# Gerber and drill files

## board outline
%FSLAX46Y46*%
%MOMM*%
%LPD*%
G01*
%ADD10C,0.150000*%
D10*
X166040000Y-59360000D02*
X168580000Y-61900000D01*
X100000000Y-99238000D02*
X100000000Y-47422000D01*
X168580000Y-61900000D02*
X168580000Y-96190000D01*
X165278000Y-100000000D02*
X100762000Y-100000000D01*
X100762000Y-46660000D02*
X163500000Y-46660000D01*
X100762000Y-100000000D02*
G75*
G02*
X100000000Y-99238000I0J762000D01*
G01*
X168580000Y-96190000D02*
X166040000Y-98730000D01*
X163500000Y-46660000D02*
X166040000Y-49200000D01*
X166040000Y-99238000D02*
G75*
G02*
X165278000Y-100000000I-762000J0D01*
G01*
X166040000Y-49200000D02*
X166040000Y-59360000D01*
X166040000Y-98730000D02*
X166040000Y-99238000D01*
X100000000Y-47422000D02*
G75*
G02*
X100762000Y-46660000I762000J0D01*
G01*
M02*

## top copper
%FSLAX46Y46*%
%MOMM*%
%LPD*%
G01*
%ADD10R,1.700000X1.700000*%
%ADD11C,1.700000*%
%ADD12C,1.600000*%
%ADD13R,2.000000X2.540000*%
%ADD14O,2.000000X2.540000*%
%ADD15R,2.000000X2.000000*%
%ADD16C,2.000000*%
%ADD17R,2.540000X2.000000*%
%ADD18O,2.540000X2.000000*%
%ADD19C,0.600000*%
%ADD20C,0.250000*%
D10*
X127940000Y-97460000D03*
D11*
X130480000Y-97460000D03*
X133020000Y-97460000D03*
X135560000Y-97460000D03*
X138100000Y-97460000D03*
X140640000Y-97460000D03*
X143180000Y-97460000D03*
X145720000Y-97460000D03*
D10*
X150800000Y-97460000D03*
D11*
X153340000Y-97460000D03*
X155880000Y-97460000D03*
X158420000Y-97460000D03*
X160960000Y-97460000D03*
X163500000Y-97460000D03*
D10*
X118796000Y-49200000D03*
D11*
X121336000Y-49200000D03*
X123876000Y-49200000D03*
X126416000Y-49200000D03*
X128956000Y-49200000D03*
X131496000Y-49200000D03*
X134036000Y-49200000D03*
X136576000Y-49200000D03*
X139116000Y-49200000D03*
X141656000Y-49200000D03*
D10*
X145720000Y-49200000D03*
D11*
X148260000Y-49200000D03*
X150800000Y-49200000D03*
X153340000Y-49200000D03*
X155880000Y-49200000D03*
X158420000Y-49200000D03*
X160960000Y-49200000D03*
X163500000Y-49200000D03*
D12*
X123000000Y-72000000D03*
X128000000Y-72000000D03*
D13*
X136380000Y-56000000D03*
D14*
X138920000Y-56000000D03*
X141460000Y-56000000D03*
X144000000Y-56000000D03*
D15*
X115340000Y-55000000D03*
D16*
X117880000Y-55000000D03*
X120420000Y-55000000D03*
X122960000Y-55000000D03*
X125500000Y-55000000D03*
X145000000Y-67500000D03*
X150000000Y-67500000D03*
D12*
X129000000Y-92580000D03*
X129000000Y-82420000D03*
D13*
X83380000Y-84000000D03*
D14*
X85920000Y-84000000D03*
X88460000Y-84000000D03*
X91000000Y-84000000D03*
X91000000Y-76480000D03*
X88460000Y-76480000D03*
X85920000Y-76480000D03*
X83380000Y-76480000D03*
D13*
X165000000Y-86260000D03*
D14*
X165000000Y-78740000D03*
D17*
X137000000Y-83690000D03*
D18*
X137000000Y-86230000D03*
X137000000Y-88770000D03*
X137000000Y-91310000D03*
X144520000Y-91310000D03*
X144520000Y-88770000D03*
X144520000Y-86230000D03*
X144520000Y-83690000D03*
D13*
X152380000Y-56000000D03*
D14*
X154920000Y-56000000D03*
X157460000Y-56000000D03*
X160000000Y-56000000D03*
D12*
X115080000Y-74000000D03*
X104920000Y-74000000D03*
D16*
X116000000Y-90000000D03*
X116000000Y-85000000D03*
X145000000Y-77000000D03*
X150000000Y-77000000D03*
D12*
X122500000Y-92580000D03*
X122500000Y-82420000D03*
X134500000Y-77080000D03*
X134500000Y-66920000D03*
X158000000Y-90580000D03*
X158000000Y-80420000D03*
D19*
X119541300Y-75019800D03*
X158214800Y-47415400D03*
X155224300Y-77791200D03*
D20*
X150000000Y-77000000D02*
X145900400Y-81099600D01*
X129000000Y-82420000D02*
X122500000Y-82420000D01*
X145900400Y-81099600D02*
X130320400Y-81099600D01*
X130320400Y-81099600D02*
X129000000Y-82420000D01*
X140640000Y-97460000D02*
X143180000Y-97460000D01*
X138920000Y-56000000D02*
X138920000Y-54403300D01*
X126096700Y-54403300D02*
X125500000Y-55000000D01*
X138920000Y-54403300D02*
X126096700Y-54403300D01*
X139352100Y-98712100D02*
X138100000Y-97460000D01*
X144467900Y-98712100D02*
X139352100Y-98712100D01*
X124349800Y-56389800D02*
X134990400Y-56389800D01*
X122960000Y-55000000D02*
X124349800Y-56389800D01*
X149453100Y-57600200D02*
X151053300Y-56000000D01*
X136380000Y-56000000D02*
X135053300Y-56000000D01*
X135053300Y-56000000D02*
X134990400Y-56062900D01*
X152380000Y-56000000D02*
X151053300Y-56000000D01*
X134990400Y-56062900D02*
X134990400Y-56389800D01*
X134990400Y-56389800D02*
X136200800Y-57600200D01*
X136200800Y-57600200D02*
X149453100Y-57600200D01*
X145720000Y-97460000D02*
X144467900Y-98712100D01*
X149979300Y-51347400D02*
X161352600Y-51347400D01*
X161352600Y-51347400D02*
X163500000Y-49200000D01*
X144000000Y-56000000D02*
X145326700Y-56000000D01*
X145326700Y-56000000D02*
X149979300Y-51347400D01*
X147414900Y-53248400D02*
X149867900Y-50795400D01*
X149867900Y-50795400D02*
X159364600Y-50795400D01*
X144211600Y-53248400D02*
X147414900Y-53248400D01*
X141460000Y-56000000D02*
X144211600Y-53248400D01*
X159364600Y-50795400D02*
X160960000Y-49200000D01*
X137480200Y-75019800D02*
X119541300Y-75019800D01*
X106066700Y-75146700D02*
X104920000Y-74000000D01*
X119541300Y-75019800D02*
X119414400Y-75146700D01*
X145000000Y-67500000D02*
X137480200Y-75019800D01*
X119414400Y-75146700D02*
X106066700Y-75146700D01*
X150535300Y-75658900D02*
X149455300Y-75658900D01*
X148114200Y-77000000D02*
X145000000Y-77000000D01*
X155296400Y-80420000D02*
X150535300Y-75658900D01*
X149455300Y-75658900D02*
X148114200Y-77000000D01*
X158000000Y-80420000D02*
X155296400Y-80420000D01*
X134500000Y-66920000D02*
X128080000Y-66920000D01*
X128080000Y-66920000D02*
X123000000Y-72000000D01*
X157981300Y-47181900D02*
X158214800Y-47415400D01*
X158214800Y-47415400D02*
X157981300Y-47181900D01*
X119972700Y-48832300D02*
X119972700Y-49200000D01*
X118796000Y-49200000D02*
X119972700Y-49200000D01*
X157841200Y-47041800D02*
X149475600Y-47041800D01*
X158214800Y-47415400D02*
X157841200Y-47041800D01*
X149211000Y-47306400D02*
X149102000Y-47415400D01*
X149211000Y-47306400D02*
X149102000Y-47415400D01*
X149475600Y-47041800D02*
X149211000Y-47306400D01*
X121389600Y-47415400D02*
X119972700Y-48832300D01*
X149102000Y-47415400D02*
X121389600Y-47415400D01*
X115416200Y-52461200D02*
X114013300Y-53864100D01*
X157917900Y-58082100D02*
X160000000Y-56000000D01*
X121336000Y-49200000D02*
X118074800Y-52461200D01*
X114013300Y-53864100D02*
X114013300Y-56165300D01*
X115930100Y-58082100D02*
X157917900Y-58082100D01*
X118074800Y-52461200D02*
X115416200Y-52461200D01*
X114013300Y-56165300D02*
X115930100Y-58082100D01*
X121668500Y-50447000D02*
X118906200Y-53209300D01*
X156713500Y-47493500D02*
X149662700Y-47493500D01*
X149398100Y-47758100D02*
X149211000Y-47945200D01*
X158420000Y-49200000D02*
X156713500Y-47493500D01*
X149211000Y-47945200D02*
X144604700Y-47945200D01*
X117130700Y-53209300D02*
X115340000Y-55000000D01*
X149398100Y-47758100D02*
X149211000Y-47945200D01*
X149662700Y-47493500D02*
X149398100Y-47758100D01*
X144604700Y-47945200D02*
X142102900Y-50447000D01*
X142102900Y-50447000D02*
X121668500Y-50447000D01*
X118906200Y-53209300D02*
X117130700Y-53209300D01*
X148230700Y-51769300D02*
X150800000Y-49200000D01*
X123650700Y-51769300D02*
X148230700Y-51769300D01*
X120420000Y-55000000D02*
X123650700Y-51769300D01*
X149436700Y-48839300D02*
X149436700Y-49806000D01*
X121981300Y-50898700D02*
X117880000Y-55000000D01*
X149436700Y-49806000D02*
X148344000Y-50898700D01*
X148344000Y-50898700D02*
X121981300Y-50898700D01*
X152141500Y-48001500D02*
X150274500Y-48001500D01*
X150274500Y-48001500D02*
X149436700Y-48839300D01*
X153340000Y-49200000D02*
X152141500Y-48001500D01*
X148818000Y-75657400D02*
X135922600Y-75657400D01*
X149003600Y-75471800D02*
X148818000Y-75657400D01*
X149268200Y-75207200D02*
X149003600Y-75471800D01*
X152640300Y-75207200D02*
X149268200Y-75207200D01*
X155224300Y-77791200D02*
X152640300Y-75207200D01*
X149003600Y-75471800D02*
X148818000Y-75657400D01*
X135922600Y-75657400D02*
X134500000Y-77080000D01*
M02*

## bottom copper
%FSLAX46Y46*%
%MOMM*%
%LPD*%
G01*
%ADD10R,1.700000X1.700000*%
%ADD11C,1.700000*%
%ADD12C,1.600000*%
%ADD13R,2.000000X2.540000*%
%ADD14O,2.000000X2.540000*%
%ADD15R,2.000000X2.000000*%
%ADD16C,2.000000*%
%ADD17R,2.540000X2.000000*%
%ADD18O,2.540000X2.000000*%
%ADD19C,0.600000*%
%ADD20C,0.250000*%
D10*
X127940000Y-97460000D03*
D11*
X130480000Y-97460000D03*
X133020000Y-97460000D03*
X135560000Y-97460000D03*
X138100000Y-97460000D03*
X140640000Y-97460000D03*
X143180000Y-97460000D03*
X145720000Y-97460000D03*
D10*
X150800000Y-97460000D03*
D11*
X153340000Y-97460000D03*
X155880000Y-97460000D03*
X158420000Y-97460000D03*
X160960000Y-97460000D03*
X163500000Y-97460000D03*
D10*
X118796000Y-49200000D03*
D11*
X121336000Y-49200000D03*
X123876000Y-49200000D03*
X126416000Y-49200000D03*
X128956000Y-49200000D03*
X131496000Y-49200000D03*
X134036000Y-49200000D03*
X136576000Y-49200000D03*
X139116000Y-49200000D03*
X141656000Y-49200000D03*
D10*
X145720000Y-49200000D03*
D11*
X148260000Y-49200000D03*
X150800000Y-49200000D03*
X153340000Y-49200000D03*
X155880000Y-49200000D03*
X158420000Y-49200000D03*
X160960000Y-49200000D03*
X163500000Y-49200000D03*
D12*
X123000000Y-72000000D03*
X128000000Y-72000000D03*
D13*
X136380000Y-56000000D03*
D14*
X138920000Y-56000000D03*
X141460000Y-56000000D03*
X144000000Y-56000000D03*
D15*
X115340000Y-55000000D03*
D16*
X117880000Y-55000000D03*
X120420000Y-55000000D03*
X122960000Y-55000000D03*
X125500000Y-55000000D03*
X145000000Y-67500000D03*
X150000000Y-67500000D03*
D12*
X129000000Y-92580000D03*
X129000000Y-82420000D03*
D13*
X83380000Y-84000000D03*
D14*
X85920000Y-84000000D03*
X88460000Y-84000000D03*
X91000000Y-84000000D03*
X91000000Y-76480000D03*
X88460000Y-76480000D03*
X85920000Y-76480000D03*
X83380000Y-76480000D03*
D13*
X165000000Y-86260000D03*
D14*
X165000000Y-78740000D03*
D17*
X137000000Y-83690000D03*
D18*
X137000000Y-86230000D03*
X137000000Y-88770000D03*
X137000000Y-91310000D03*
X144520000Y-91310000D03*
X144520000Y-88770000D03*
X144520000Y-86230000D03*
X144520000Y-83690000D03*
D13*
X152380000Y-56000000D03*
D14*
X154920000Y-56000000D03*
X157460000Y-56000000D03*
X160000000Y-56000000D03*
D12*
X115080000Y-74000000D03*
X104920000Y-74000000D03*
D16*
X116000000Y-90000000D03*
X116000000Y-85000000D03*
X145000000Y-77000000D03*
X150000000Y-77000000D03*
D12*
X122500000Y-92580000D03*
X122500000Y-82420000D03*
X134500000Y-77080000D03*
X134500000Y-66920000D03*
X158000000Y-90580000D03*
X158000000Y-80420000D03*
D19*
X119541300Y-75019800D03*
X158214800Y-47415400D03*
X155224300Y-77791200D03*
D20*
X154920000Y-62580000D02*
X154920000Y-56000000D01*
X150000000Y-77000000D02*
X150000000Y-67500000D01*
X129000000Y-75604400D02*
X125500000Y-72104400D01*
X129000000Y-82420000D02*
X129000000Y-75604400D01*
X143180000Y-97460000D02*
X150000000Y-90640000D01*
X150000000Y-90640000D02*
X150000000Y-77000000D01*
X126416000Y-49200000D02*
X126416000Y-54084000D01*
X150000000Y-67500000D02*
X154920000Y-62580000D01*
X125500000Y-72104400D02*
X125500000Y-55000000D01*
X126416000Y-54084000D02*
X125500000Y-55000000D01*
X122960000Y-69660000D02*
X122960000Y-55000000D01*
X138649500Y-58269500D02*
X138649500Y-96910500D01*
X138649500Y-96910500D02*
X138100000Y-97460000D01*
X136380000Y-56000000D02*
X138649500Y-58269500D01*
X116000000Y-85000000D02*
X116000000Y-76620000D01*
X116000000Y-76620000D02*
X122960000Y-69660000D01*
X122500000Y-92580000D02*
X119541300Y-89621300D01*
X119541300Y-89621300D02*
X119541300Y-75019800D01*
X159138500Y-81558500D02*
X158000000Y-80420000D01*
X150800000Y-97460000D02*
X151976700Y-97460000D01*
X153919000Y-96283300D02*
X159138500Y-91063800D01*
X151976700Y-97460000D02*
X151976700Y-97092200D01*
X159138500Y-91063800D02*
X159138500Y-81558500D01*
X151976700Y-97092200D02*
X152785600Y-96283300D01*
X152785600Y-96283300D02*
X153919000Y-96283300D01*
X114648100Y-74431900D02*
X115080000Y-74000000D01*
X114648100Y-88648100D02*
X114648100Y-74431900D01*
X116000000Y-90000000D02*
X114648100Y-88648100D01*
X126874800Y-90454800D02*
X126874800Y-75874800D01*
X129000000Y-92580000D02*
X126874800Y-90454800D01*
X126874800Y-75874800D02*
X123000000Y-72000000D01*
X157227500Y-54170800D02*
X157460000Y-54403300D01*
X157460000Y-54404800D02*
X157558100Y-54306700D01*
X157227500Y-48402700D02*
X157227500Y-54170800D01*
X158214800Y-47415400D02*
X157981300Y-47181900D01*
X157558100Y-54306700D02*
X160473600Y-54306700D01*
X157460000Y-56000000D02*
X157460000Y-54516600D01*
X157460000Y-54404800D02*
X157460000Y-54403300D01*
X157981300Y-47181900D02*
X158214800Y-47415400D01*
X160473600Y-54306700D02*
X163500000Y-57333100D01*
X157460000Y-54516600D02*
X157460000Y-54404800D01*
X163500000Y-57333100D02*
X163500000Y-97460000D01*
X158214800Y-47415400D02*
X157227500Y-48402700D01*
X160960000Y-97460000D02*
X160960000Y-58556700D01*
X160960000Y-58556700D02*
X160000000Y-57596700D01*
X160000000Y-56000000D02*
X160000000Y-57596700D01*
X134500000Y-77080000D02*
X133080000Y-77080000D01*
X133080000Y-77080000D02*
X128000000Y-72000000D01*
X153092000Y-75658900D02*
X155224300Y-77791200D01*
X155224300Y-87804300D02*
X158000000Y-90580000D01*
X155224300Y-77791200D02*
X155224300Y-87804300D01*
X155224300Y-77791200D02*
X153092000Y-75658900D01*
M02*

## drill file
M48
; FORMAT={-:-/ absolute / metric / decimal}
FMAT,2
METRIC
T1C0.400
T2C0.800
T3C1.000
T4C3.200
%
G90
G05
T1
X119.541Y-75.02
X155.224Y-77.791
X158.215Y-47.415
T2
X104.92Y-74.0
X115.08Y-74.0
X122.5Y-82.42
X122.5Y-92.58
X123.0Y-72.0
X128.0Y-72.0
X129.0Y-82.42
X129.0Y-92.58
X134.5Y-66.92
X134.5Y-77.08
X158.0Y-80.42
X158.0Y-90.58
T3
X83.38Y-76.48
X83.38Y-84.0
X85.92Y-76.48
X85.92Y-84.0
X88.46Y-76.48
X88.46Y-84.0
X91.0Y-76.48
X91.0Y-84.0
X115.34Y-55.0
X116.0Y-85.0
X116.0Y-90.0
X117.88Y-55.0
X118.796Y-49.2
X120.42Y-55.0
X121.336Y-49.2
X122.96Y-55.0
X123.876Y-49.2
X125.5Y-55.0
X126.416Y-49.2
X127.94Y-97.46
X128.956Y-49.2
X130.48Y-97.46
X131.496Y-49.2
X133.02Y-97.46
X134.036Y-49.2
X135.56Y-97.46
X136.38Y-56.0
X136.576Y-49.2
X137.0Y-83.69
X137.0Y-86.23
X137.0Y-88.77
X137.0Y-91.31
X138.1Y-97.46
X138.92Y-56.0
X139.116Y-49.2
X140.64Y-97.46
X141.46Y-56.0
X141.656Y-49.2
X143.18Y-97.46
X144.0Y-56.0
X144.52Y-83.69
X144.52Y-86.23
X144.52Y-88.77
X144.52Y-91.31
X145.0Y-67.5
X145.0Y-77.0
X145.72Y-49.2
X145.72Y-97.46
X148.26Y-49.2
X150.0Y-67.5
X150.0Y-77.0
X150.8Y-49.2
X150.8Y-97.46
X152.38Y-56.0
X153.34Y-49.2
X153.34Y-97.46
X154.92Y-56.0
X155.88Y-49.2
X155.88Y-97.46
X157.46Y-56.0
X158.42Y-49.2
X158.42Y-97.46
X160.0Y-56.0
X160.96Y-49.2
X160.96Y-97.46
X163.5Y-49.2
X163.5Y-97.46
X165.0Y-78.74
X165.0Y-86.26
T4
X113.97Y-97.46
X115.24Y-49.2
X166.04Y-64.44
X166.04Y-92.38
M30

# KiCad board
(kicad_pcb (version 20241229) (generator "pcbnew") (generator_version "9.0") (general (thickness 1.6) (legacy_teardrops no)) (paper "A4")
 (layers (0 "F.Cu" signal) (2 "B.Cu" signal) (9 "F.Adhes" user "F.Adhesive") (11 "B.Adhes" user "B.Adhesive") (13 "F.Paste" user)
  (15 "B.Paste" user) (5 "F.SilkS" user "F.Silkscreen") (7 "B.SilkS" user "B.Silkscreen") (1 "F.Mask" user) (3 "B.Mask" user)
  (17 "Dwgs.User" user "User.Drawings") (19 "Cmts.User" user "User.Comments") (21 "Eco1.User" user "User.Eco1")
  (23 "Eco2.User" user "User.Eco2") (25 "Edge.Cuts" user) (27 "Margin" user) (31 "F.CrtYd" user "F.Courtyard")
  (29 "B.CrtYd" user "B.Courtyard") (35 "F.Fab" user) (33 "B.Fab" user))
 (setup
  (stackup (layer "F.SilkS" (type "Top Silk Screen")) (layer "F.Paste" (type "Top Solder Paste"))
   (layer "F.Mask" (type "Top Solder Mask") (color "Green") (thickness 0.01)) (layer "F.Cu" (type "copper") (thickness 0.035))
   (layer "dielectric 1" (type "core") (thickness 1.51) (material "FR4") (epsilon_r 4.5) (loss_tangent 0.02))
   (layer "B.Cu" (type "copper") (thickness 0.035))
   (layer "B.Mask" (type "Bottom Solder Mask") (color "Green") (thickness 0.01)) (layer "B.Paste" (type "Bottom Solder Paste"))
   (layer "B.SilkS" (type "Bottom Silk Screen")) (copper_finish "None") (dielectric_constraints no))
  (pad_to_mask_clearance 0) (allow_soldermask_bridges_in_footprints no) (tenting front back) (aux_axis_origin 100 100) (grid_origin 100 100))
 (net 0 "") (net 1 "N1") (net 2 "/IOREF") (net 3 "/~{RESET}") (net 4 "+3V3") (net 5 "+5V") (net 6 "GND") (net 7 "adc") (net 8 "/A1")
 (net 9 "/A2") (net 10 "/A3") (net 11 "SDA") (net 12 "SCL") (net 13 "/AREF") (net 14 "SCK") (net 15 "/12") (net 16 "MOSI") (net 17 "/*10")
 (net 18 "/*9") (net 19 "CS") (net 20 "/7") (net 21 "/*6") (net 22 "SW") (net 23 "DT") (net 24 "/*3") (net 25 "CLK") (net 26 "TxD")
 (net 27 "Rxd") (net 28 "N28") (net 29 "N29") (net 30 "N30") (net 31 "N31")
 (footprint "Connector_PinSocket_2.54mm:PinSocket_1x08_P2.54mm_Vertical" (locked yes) (layer "F.Cu") (at 127.94 97.46 90)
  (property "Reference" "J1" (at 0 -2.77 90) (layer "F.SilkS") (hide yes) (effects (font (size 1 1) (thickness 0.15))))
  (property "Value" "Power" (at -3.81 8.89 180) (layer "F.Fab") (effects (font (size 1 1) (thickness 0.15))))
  (pad "1" thru_hole rect (at 0 0 90) (size 1.7 1.7) (drill 1) (layers "*.Cu" "*.Mask") (remove_unused_layers no) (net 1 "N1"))
  (pad "2" thru_hole circle (at 0 2.54 90) (size 1.7 1.7) (drill 1) (layers "*.Cu" "*.Mask") (remove_unused_layers no) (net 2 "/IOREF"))
  (pad "3" thru_hole circle (at 0 5.08 90) (size 1.7 1.7) (drill 1) (layers "*.Cu" "*.Mask") (remove_unused_layers no) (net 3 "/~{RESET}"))
  (pad "4" thru_hole circle (at 0 7.62 90) (size 1.7 1.7) (drill 1) (layers "*.Cu" "*.Mask") (remove_unused_layers no) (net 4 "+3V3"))
  (pad "5" thru_hole circle (at 0 10.16 90) (size 1.7 1.7) (drill 1) (layers "*.Cu" "*.Mask") (remove_unused_layers no) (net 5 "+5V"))
  (pad "6" thru_hole circle (at 0 12.7 90) (size 1.7 1.7) (drill 1) (layers "*.Cu" "*.Mask") (remove_unused_layers no) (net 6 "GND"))
  (pad "7" thru_hole circle (at 0 15.24 90) (size 1.7 1.7) (drill 1) (layers "*.Cu" "*.Mask") (remove_unused_layers no) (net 6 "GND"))
  (pad "8" thru_hole circle (at 0 17.78 90) (size 1.7 1.7) (drill 1) (layers "*.Cu" "*.Mask") (remove_unused_layers no) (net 5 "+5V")))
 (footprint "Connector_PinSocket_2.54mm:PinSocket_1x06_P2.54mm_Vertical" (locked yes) (layer "F.Cu") (at 150.8 97.46 90)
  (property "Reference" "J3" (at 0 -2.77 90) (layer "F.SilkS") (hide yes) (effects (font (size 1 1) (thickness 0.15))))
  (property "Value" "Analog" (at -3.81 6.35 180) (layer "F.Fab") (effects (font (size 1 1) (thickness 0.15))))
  (pad "1" thru_hole rect (at 0 0 90) (size 1.7 1.7) (drill 1) (layers "*.Cu" "*.Mask") (remove_unused_layers no) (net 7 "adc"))
  (pad "2" thru_hole circle (at 0 2.54 90) (size 1.7 1.7) (drill 1) (layers "*.Cu" "*.Mask") (remove_unused_layers no) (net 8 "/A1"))
  (pad "3" thru_hole circle (at 0 5.08 90) (size 1.7 1.7) (drill 1) (layers "*.Cu" "*.Mask") (remove_unused_layers no) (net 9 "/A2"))
  (pad "4" thru_hole circle (at 0 7.62 90) (size 1.7 1.7) (drill 1) (layers "*.Cu" "*.Mask") (remove_unused_layers no) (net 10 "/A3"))
  (pad "5" thru_hole circle (at 0 10.16 90) (size 1.7 1.7) (drill 1) (layers "*.Cu" "*.Mask") (remove_unused_layers no) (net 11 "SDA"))
  (pad "6" thru_hole circle (at 0 12.7 90) (size 1.7 1.7) (drill 1) (layers "*.Cu" "*.Mask") (remove_unused_layers no) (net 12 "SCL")))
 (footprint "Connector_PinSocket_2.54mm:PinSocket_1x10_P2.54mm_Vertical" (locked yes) (layer "F.Cu") (at 118.796 49.2 90)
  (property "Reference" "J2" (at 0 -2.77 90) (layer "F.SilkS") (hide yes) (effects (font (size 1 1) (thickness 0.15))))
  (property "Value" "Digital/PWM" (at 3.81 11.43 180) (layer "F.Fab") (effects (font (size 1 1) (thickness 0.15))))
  (pad "1" thru_hole rect (at 0 0 90) (size 1.7 1.7) (drill 1) (layers "*.Cu" "*.Mask") (remove_unused_layers no) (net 12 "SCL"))
  (pad "2" thru_hole circle (at 0 2.54 90) (size 1.7 1.7) (drill 1) (layers "*.Cu" "*.Mask") (remove_unused_layers no) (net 11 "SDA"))
  (pad "3" thru_hole circle (at 0 5.08 90) (size 1.7 1.7) (drill 1) (layers "*.Cu" "*.Mask") (remove_unused_layers no) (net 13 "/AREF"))
  (pad "4" thru_hole circle (at 0 7.62 90) (size 1.7 1.7) (drill 1) (layers "*.Cu" "*.Mask") (remove_unused_layers no) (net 6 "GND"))
  (pad "5" thru_hole circle (at 0 10.16 90) (size 1.7 1.7) (drill 1) (layers "*.Cu" "*.Mask") (remove_unused_layers no) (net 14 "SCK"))
  (pad "6" thru_hole circle (at 0 12.7 90) (size 1.7 1.7) (drill 1) (layers "*.Cu" "*.Mask") (remove_unused_layers no) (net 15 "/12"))
  (pad "7" thru_hole circle (at 0 15.24 90) (size 1.7 1.7) (drill 1) (layers "*.Cu" "*.Mask") (remove_unused_layers no) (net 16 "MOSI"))
  (pad "8" thru_hole circle (at 0 17.78 90) (size 1.7 1.7) (drill 1) (layers "*.Cu" "*.Mask") (remove_unused_layers no) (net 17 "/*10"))
  (pad "9" thru_hole circle (at 0 20.32 90) (size 1.7 1.7) (drill 1) (layers "*.Cu" "*.Mask") (remove_unused_layers no) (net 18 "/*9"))
  (pad "10" thru_hole circle (at 0 22.86 90) (size 1.7 1.7) (drill 1) (layers "*.Cu" "*.Mask") (remove_unused_layers no) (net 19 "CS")))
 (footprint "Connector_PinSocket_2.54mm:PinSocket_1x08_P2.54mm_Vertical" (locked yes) (layer "F.Cu") (at 145.72 49.2 90)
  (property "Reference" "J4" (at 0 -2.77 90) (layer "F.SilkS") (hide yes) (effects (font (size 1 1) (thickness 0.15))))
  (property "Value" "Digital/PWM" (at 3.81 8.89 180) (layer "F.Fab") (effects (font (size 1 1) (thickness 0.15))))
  (pad "1" thru_hole rect (at 0 0 90) (size 1.7 1.7) (drill 1) (layers "*.Cu" "*.Mask") (remove_unused_layers no) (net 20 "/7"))
  (pad "2" thru_hole circle (at 0 2.54 90) (size 1.7 1.7) (drill 1) (layers "*.Cu" "*.Mask") (remove_unused_layers no) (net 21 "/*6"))
  (pad "3" thru_hole circle (at 0 5.08 90) (size 1.7 1.7) (drill 1) (layers "*.Cu" "*.Mask") (remove_unused_layers no) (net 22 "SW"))
  (pad "4" thru_hole circle (at 0 7.62 90) (size 1.7 1.7) (drill 1) (layers "*.Cu" "*.Mask") (remove_unused_layers no) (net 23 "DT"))
  (pad "5" thru_hole circle (at 0 10.16 90) (size 1.7 1.7) (drill 1) (layers "*.Cu" "*.Mask") (remove_unused_layers no) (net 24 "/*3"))
  (pad "6" thru_hole circle (at 0 12.7 90) (size 1.7 1.7) (drill 1) (layers "*.Cu" "*.Mask") (remove_unused_layers no) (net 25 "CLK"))
  (pad "7" thru_hole circle (at 0 15.24 90) (size 1.7 1.7) (drill 1) (layers "*.Cu" "*.Mask") (remove_unused_layers no) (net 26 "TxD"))
  (pad "8" thru_hole circle (at 0 17.78 90) (size 1.7 1.7) (drill 1) (layers "*.Cu" "*.Mask") (remove_unused_layers no) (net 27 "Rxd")))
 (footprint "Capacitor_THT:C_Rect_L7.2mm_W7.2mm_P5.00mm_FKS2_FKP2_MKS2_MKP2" (layer "F.Cu") (at 123 72)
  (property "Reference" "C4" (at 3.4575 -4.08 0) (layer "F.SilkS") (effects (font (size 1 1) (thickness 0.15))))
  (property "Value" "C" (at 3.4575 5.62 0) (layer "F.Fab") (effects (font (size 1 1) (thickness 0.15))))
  (pad "1" thru_hole circle (at 0 0) (size 1.6 1.6) (drill 0.8) (layers "*.Cu" "*.Mask") (remove_unused_layers no) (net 6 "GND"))
  (pad "2" thru_hole circle (at 5 0) (size 1.6 1.6) (drill 0.8) (layers "*.Cu" "*.Mask") (remove_unused_layers no) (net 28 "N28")))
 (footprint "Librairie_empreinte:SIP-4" (layer "F.Cu") (at 140.19 56)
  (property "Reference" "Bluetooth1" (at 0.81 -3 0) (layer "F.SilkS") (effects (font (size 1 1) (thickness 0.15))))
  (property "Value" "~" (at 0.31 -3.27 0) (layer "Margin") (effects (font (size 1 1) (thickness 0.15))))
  (pad "1" thru_hole rect (at -3.81 0) (size 2 2.54) (drill 1) (layers "*.Cu" "*.Mask") (remove_unused_layers no) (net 5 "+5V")
   (thermal_bridge_angle 45))
  (pad "2" thru_hole oval (at -1.27 0) (size 2 2.54) (drill 1) (layers "*.Cu" "*.Mask") (remove_unused_layers no) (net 6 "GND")
   (thermal_bridge_angle 45))
  (pad "3" thru_hole oval (at 1.27 0) (size 2 2.54) (drill 1) (layers "*.Cu" "*.Mask") (remove_unused_layers no) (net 26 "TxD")
   (thermal_bridge_angle 45))
  (pad "4" thru_hole oval (at 3.81 0) (size 2 2.54) (drill 1) (layers "*.Cu" "*.Mask") (remove_unused_layers no) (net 27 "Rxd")
   (thermal_bridge_angle 45)))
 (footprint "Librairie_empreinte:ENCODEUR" (layer "F.Cu") (at 120.42 55)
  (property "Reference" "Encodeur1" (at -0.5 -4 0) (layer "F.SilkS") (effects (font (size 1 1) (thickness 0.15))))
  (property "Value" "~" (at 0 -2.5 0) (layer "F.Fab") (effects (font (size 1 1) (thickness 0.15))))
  (pad "1" thru_hole rect (at -5.08 0) (size 2 2) (drill 1) (layers "*.Cu" "*.Mask") (remove_unused_layers no) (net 25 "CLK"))
  (pad "2" thru_hole circle (at -2.54 0) (size 2 2) (drill 1) (layers "*.Cu" "*.Mask") (remove_unused_layers no) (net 23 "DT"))
  (pad "3" thru_hole circle (at 0 0) (size 2 2) (drill 1) (layers "*.Cu" "*.Mask") (remove_unused_layers no) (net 22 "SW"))
  (pad "4" thru_hole circle (at 2.54 0) (size 2 2) (drill 1) (layers "*.Cu" "*.Mask") (remove_unused_layers no) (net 5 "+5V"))
  (pad "5" thru_hole circle (at 5.08 0) (size 2 2) (drill 1) (layers "*.Cu" "*.Mask") (remove_unused_layers no) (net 6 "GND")))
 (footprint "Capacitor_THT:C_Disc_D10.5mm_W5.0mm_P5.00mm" (layer "F.Cu") (at 145 67.5)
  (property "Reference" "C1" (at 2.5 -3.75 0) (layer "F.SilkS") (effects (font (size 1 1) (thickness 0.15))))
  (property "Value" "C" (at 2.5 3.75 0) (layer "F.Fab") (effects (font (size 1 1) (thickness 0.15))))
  (pad "1" thru_hole circle (at 0 0) (size 2 2) (drill 1) (layers "*.Cu" "*.Mask") (remove_unused_layers no) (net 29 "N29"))
  (pad "2" thru_hole circle (at 5 0) (size 2 2) (drill 1) (layers "*.Cu" "*.Mask") (remove_unused_layers no) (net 6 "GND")))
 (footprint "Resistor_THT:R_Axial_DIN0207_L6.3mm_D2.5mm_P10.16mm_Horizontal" (layer "F.Cu") (at 129 92.58 90)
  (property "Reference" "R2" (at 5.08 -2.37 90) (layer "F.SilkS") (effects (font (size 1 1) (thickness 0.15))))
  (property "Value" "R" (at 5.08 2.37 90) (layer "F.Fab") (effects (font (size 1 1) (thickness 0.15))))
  (pad "1" thru_hole circle (at 0 0 90) (size 1.6 1.6) (drill 0.8) (layers "*.Cu" "*.Mask") (remove_unused_layers no) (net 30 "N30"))
  (pad "2" thru_hole circle (at 10.16 0 90) (size 1.6 1.6) (drill 0.8) (layers "*.Cu" "*.Mask") (remove_unused_layers no) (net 6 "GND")))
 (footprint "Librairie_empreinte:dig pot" (layer "F.Cu") (at 87.19 80.24)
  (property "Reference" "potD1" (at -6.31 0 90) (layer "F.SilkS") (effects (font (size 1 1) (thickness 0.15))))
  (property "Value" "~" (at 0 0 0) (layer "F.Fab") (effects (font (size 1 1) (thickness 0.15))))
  (pad "1" thru_hole rect (at -3.81 3.76) (size 2 2.54) (drill 1) (layers "*.Cu" "*.Mask") (remove_unused_layers no)
   (thermal_bridge_angle 45))
  (pad "2" thru_hole oval (at -1.27 3.76) (size 2 2.54) (drill 1) (layers "*.Cu" "*.Mask") (remove_unused_layers no)
   (thermal_bridge_angle 45))
  (pad "3" thru_hole oval (at 1.27 3.76) (size 2 2.54) (drill 1) (layers "*.Cu" "*.Mask") (remove_unused_layers no)
   (thermal_bridge_angle 45))
  (pad "4" thru_hole oval (at 3.81 3.76) (size 2 2.54) (drill 1) (layers "*.Cu" "*.Mask") (remove_unused_layers no)
   (thermal_bridge_angle 45))
  (pad "5" thru_hole oval (at 3.81 -3.76) (size 2 2.54) (drill 1) (layers "*.Cu" "*.Mask") (remove_unused_layers no)
   (thermal_bridge_angle 45))
  (pad "6" thru_hole oval (at 1.27 -3.76) (size 2 2.54) (drill 1) (layers "*.Cu" "*.Mask") (remove_unused_layers no)
   (thermal_bridge_angle 45))
  (pad "7" thru_hole oval (at -1.27 -3.76) (size 2 2.54) (drill 1) (layers "*.Cu" "*.Mask") (remove_unused_layers no)
   (thermal_bridge_angle 45))
  (pad "8" thru_hole oval (at -3.81 -3.76) (size 2 2.54) (drill 1) (layers "*.Cu" "*.Mask") (remove_unused_layers no)
   (thermal_bridge_angle 45)))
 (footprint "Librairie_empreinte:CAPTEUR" (layer "F.Cu") (at 165 82.5)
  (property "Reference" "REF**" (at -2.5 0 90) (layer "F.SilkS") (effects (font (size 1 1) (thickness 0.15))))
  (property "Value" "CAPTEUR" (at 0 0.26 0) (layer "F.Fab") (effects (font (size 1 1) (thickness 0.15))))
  (pad "1" thru_hole rect (at 0 3.76) (size 2 2.54) (drill 1) (layers "*.Cu" "*.Mask") (remove_unused_layers no) (thermal_bridge_angle 45))
  (pad "2" thru_hole oval (at 0 -3.76) (size 2 2.54) (drill 1) (layers "*.Cu" "*.Mask") (remove_unused_layers no) (thermal_bridge_angle 45)))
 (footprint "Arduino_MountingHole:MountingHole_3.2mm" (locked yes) (layer "F.Cu") (at 115.24 49.2)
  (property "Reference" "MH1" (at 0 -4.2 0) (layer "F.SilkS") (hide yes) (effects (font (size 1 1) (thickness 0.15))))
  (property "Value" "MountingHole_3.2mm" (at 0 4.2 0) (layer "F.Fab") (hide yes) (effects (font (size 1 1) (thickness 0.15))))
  (pad "" np_thru_hole circle (at 0 0) (size 3.2 3.2) (drill 3.2) (layers "*.Cu" "*.Mask")))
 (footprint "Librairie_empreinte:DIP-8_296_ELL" (layer "F.Cu") (at 140.76 87.5 -90)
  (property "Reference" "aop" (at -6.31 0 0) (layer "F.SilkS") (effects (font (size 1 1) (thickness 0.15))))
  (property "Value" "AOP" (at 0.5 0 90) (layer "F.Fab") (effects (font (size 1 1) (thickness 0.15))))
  (pad "1" thru_hole rect (at -3.81 3.76 270) (size 2 2.54) (drill 1) (layers "*.Cu" "*.Mask") (remove_unused_layers no)
   (thermal_bridge_angle 45))
  (pad "2" thru_hole oval (at -1.27 3.76 270) (size 2 2.54) (drill 1) (layers "*.Cu" "*.Mask") (remove_unused_layers no)
   (thermal_bridge_angle 45))
  (pad "3" thru_hole oval (at 1.27 3.76 270) (size 2 2.54) (drill 1) (layers "*.Cu" "*.Mask") (remove_unused_layers no)
   (thermal_bridge_angle 45))
  (pad "4" thru_hole oval (at 3.81 3.76 270) (size 2 2.54) (drill 1) (layers "*.Cu" "*.Mask") (remove_unused_layers no)
   (thermal_bridge_angle 45))
  (pad "5" thru_hole oval (at 3.81 -3.76 270) (size 2 2.54) (drill 1) (layers "*.Cu" "*.Mask") (remove_unused_layers no)
   (thermal_bridge_angle 45))
  (pad "6" thru_hole oval (at 1.27 -3.76 270) (size 2 2.54) (drill 1) (layers "*.Cu" "*.Mask") (remove_unused_layers no)
   (thermal_bridge_angle 45))
  (pad "7" thru_hole oval (at -1.27 -3.76 270) (size 2 2.54) (drill 1) (layers "*.Cu" "*.Mask") (remove_unused_layers no)
   (thermal_bridge_angle 45))
  (pad "8" thru_hole oval (at -3.81 -3.76 270) (size 2 2.54) (drill 1) (layers "*.Cu" "*.Mask") (remove_unused_layers no)
   (thermal_bridge_angle 45)))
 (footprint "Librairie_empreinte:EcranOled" (layer "F.Cu") (at 156.19 56)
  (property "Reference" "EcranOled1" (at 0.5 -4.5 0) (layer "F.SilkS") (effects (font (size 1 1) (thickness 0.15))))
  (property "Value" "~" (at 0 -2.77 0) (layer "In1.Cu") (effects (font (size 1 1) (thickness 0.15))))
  (pad "1" thru_hole rect (at -3.81 0) (size 2 2.54) (drill 1) (layers "*.Cu" "*.Mask") (remove_unused_layers no) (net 5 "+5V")
   (thermal_bridge_angle 45))
  (pad "2" thru_hole oval (at -1.27 0) (size 2 2.54) (drill 1) (layers "*.Cu" "*.Mask") (remove_unused_layers no) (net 6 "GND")
   (thermal_bridge_angle 45))
  (pad "3" thru_hole oval (at 1.27 0) (size 2 2.54) (drill 1) (layers "*.Cu" "*.Mask") (remove_unused_layers no) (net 12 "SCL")
   (thermal_bridge_angle 45))
  (pad "4" thru_hole oval (at 3.81 0) (size 2 2.54) (drill 1) (layers "*.Cu" "*.Mask") (remove_unused_layers no) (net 11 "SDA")
   (thermal_bridge_angle 45)))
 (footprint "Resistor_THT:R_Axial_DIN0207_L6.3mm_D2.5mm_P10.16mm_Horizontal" (layer "F.Cu") (at 115.08 74 180)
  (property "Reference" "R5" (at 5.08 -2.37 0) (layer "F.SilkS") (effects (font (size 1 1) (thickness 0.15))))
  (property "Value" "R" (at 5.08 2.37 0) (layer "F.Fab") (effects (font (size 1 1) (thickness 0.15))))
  (pad "1" thru_hole circle (at 0 0 180) (size 1.6 1.6) (drill 0.8) (layers "*.Cu" "*.Mask") (remove_unused_layers no) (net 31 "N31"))
  (pad "2" thru_hole circle (at 10.16 0 180) (size 1.6 1.6) (drill 0.8) (layers "*.Cu" "*.Mask") (remove_unused_layers no) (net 29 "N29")))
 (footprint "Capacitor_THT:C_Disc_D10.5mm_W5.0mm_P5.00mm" (layer "F.Cu") (at 116 90 90)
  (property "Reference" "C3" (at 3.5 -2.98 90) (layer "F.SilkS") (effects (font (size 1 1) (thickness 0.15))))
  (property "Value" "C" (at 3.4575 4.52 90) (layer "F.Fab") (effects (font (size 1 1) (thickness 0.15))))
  (pad "1" thru_hole circle (at 0 0 90) (size 2 2) (drill 1) (layers "*.Cu" "*.Mask") (remove_unused_layers no) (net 31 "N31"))
  (pad "2" thru_hole circle (at 5 0 90) (size 2 2) (drill 1) (layers "*.Cu" "*.Mask") (remove_unused_layers no) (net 5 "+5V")))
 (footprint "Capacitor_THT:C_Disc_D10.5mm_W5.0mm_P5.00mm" (layer "F.Cu") (at 145 77)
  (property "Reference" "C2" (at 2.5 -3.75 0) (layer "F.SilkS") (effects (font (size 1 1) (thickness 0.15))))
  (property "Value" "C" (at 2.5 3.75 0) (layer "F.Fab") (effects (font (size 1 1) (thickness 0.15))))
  (pad "1" thru_hole circle (at 0 0) (size 2 2) (drill 1) (layers "*.Cu" "*.Mask") (remove_unused_layers no) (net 7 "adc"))
  (pad "2" thru_hole circle (at 5 0) (size 2 2) (drill 1) (layers "*.Cu" "*.Mask") (remove_unused_layers no) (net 6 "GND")))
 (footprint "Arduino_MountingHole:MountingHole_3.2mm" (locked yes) (layer "F.Cu") (at 113.97 97.46)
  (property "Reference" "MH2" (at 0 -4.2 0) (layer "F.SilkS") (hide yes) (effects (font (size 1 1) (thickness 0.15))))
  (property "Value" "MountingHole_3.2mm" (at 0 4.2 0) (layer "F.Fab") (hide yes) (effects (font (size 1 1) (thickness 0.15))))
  (pad "" np_thru_hole circle (at 0 0) (size 3.2 3.2) (drill 3.2) (layers "*.Cu" "*.Mask")))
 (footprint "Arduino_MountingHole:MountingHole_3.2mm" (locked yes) (layer "F.Cu") (at 166.04 64.44)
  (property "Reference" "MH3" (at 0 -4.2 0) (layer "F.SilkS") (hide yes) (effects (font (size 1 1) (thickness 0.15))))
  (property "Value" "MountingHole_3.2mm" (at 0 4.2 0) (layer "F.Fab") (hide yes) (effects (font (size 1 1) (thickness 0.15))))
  (pad "" np_thru_hole circle (at 0 0) (size 3.2 3.2) (drill 3.2) (layers "*.Cu" "*.Mask")))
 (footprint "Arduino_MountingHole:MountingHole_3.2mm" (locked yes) (layer "F.Cu") (at 166.04 92.38)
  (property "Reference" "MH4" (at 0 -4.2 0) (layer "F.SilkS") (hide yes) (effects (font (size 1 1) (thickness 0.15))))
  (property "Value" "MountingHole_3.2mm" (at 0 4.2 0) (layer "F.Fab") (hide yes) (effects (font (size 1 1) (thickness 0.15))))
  (pad "" np_thru_hole circle (at 0 0) (size 3.2 3.2) (drill 3.2) (layers "*.Cu" "*.Mask")))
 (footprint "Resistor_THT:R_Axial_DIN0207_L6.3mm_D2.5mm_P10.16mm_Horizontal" (layer "F.Cu") (at 122.5 92.58 90)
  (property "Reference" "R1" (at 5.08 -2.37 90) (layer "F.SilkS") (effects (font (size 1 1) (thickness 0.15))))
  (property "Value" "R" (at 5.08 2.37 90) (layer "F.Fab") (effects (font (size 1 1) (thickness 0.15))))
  (pad "1" thru_hole circle (at 0 0 90) (size 1.6 1.6) (drill 0.8) (layers "*.Cu" "*.Mask") (remove_unused_layers no) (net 29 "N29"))
  (pad "2" thru_hole circle (at 10.16 0 90) (size 1.6 1.6) (drill 0.8) (layers "*.Cu" "*.Mask") (remove_unused_layers no) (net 6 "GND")))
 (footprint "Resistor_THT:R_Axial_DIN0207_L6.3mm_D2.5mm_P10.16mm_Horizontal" (layer "F.Cu") (at 134.5 77.08 90)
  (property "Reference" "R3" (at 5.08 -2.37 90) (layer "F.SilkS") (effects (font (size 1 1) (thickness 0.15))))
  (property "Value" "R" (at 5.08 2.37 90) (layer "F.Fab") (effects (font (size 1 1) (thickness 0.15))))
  (pad "1" thru_hole circle (at 0 0 90) (size 1.6 1.6) (drill 0.8) (layers "*.Cu" "*.Mask") (remove_unused_layers no) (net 28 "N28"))
  (pad "2" thru_hole circle (at 10.16 0 90) (size 1.6 1.6) (drill 0.8) (layers "*.Cu" "*.Mask") (remove_unused_layers no) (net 6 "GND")))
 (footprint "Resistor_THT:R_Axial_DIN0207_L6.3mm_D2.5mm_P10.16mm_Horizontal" (layer "F.Cu") (at 158 90.58 90)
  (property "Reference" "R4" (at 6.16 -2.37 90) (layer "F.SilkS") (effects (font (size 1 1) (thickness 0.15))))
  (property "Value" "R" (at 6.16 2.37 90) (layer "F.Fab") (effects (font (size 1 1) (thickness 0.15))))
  (pad "1" thru_hole circle (at 0 0 90) (size 1.6 1.6) (drill 0.8) (layers "*.Cu" "*.Mask") (remove_unused_layers no) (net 28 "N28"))
  (pad "2" thru_hole circle (at 10.16 0 90) (size 1.6 1.6) (drill 0.8) (layers "*.Cu" "*.Mask") (remove_unused_layers no) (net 7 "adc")))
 (gr_line (start 166.04 59.36) (end 168.58 61.9) (stroke (width 0.15) (type solid)) (layer "Edge.Cuts"))
 (gr_line (start 100 99.238) (end 100 47.422) (stroke (width 0.15) (type solid)) (layer "Edge.Cuts"))
 (gr_line (start 168.58 61.9) (end 168.58 96.19) (stroke (width 0.15) (type solid)) (layer "Edge.Cuts"))
 (gr_line (start 165.278 100) (end 100.762 100) (stroke (width 0.15) (type solid)) (layer "Edge.Cuts"))
 (gr_line (start 100.762 46.66) (end 163.5 46.66) (stroke (width 0.15) (type solid)) (layer "Edge.Cuts"))
 (gr_arc (start 100.762 100) (mid 100.223185 99.776815) (end 100 99.238) (stroke (width 0.15) (type solid)) (layer "Edge.Cuts"))
 (gr_line (start 168.58 96.19) (end 166.04 98.73) (stroke (width 0.15) (type solid)) (layer "Edge.Cuts"))
 (gr_line (start 163.5 46.66) (end 166.04 49.2) (stroke (width 0.15) (type solid)) (layer "Edge.Cuts"))
 (gr_arc (start 166.04 99.238) (mid 165.816815 99.776815) (end 165.278 100) (stroke (width 0.15) (type solid)) (layer "Edge.Cuts"))
 (gr_line (start 166.04 49.2) (end 166.04 59.36) (stroke (width 0.15) (type solid)) (layer "Edge.Cuts"))
 (gr_line (start 166.04 98.73) (end 166.04 99.238) (stroke (width 0.15) (type solid)) (layer "Edge.Cuts"))
 (gr_arc (start 100 47.422) (mid 100.223185 46.883185) (end 100.762 46.66) (stroke (width 0.15) (type solid)) (layer "Edge.Cuts"))
 (segment (start 150 77) (end 145.9004 81.0996) (width 0.25) (layer "F.Cu") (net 6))
 (segment (start 129 82.42) (end 122.5 82.42) (width 0.25) (layer "F.Cu") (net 6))
 (segment (start 145.9004 81.0996) (end 130.3204 81.0996) (width 0.25) (layer "F.Cu") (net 6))
 (segment (start 130.3204 81.0996) (end 129 82.42) (width 0.25) (layer "F.Cu") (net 6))
 (segment (start 140.64 97.46) (end 143.18 97.46) (width 0.25) (layer "F.Cu") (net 6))
 (segment (start 138.92 56) (end 138.92 54.4033) (width 0.25) (layer "F.Cu") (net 6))
 (segment (start 126.0967 54.4033) (end 125.5 55) (width 0.25) (layer "F.Cu") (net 6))
 (segment (start 138.92 54.4033) (end 126.0967 54.4033) (width 0.25) (layer "F.Cu") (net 6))
 (segment (start 154.92 62.58) (end 154.92 56) (width 0.25) (layer "B.Cu") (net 6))
 (segment (start 150 77) (end 150 67.5) (width 0.25) (layer "B.Cu") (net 6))
 (segment (start 129 75.6044) (end 125.5 72.1044) (width 0.25) (layer "B.Cu") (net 6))
 (segment (start 129 82.42) (end 129 75.6044) (width 0.25) (layer "B.Cu") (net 6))
 (segment (start 143.18 97.46) (end 150 90.64) (width 0.25) (layer "B.Cu") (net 6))
 (segment (start 150 90.64) (end 150 77) (width 0.25) (layer "B.Cu") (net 6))
 (segment (start 126.416 49.2) (end 126.416 54.084) (width 0.25) (layer "B.Cu") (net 6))
 (segment (start 150 67.5) (end 154.92 62.58) (width 0.25) (layer "B.Cu") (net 6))
 (segment (start 125.5 72.1044) (end 125.5 55) (width 0.25) (layer "B.Cu") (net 6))
 (segment (start 126.416 54.084) (end 125.5 55) (width 0.25) (layer "B.Cu") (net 6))
 (segment (start 139.3521 98.7121) (end 138.1 97.46) (width 0.25) (layer "F.Cu") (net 5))
 (segment (start 144.4679 98.7121) (end 139.3521 98.7121) (width 0.25) (layer "F.Cu") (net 5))
 (segment (start 124.3498 56.3898) (end 134.9904 56.3898) (width 0.25) (layer "F.Cu") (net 5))
 (segment (start 122.96 55) (end 124.3498 56.3898) (width 0.25) (layer "F.Cu") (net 5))
 (segment (start 149.4531 57.6002) (end 151.0533 56) (width 0.25) (layer "F.Cu") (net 5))
 (segment (start 136.38 56) (end 135.0533 56) (width 0.25) (layer "F.Cu") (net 5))
 (segment (start 135.0533 56) (end 134.9904 56.0629) (width 0.25) (layer "F.Cu") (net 5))
 (segment (start 152.38 56) (end 151.0533 56) (width 0.25) (layer "F.Cu") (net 5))
 (segment (start 134.9904 56.0629) (end 134.9904 56.3898) (width 0.25) (layer "F.Cu") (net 5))
 (segment (start 134.9904 56.3898) (end 136.2008 57.6002) (width 0.25) (layer "F.Cu") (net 5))
 (segment (start 136.2008 57.6002) (end 149.4531 57.6002) (width 0.25) (layer "F.Cu") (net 5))
 (segment (start 145.72 97.46) (end 144.4679 98.7121) (width 0.25) (layer "F.Cu") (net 5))
 (segment (start 122.96 69.66) (end 122.96 55) (width 0.25) (layer "B.Cu") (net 5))
 (segment (start 138.6495 58.2695) (end 138.6495 96.9105) (width 0.25) (layer "B.Cu") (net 5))
 (segment (start 138.6495 96.9105) (end 138.1 97.46) (width 0.25) (layer "B.Cu") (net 5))
 (segment (start 136.38 56) (end 138.6495 58.2695) (width 0.25) (layer "B.Cu") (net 5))
 (segment (start 116 85) (end 116 76.62) (width 0.25) (layer "B.Cu") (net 5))
 (segment (start 116 76.62) (end 122.96 69.66) (width 0.25) (layer "B.Cu") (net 5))
 (segment (start 149.9793 51.3474) (end 161.3526 51.3474) (width 0.25) (layer "F.Cu") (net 27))
 (segment (start 161.3526 51.3474) (end 163.5 49.2) (width 0.25) (layer "F.Cu") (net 27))
 (segment (start 144 56) (end 145.3267 56) (width 0.25) (layer "F.Cu") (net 27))
 (segment (start 145.3267 56) (end 149.9793 51.3474) (width 0.25) (layer "F.Cu") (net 27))
 (segment (start 147.4149 53.2484) (end 149.8679 50.7954) (width 0.25) (layer "F.Cu") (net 26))
 (segment (start 149.8679 50.7954) (end 159.3646 50.7954) (width 0.25) (layer "F.Cu") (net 26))
 (segment (start 144.2116 53.2484) (end 147.4149 53.2484) (width 0.25) (layer "F.Cu") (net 26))
 (segment (start 141.46 56) (end 144.2116 53.2484) (width 0.25) (layer "F.Cu") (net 26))
 (segment (start 159.3646 50.7954) (end 160.96 49.2) (width 0.25) (layer "F.Cu") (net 26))
 (segment (start 137.4802 75.0198) (end 119.5413 75.0198) (width 0.25) (layer "F.Cu") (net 29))
 (segment (start 106.0667 75.1467) (end 104.92 74) (width 0.25) (layer "F.Cu") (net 29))
 (segment (start 119.5413 75.0198) (end 119.4144 75.1467) (width 0.25) (layer "F.Cu") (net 29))
 (segment (start 145 67.5) (end 137.4802 75.0198) (width 0.25) (layer "F.Cu") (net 29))
 (segment (start 119.4144 75.1467) (end 106.0667 75.1467) (width 0.25) (layer "F.Cu") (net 29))
 (via (at 119.5413 75.0198) (size 0.6) (drill 0.4) (layers "F.Cu" "B.Cu") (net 29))
 (segment (start 122.5 92.58) (end 119.5413 89.6213) (width 0.25) (layer "B.Cu") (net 29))
 (segment (start 119.5413 89.6213) (end 119.5413 75.0198) (width 0.25) (layer "B.Cu") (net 29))
 (segment (start 150.5353 75.6589) (end 149.4553 75.6589) (width 0.25) (layer "F.Cu") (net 7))
 (segment (start 148.1142 77) (end 145 77) (width 0.25) (layer "F.Cu") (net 7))
 (segment (start 155.2964 80.42) (end 150.5353 75.6589) (width 0.25) (layer "F.Cu") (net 7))
 (segment (start 149.4553 75.6589) (end 148.1142 77) (width 0.25) (layer "F.Cu") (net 7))
 (segment (start 158 80.42) (end 155.2964 80.42) (width 0.25) (layer "F.Cu") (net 7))
 (segment (start 159.1385 81.5585) (end 158 80.42) (width 0.25) (layer "B.Cu") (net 7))
 (segment (start 150.8 97.46) (end 151.9767 97.46) (width 0.25) (layer "B.Cu") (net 7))
 (segment (start 153.919 96.2833) (end 159.1385 91.0638) (width 0.25) (layer "B.Cu") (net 7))
 (segment (start 151.9767 97.46) (end 151.9767 97.0922) (width 0.25) (layer "B.Cu") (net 7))
 (segment (start 159.1385 91.0638) (end 159.1385 81.5585) (width 0.25) (layer "B.Cu") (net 7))
 (segment (start 151.9767 97.0922) (end 152.7856 96.2833) (width 0.25) (layer "B.Cu") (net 7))
 (segment (start 152.7856 96.2833) (end 153.919 96.2833) (width 0.25) (layer "B.Cu") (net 7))
 (segment (start 114.6481 74.4319) (end 115.08 74) (width 0.25) (layer "B.Cu") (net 31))
 (segment (start 114.6481 88.6481) (end 114.6481 74.4319) (width 0.25) (layer "B.Cu") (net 31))
 (segment (start 116 90) (end 114.6481 88.6481) (width 0.25) (layer "B.Cu") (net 31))
 (segment (start 134.5 66.92) (end 128.08 66.92) (width 0.25) (layer "F.Cu") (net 30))
 (segment (start 128.08 66.92) (end 123 72) (width 0.25) (layer "F.Cu") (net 30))
 (segment (start 126.8748 90.4548) (end 126.8748 75.8748) (width 0.25) (layer "B.Cu") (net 30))
 (segment (start 129 92.58) (end 126.8748 90.4548) (width 0.25) (layer "B.Cu") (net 30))
 (segment (start 126.8748 75.8748) (end 123 72) (width 0.25) (layer "B.Cu") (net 30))
 (segment (start 157.9813 47.1819) (end 158.2148 47.4154) (width 0.25) (layer "F.Cu") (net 12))
 (segment (start 158.2148 47.4154) (end 157.9813 47.1819) (width 0.25) (layer "F.Cu") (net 12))
 (segment (start 119.9727 48.8323) (end 119.9727 49.2) (width 0.25) (layer "F.Cu") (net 12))
 (segment (start 118.796 49.2) (end 119.9727 49.2) (width 0.25) (layer "F.Cu") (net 12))
 (segment (start 157.8412 47.0418) (end 149.4756 47.0418) (width 0.25) (layer "F.Cu") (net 12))
 (segment (start 158.2148 47.4154) (end 157.8412 47.0418) (width 0.25) (layer "F.Cu") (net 12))
 (segment (start 149.211 47.3064) (end 149.102 47.4154) (width 0.25) (layer "F.Cu") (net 12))
 (segment (start 149.211 47.3064) (end 149.102 47.4154) (width 0.25) (layer "F.Cu") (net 12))
 (segment (start 149.4756 47.0418) (end 149.211 47.3064) (width 0.25) (layer "F.Cu") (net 12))
 (segment (start 121.3896 47.4154) (end 119.9727 48.8323) (width 0.25) (layer "F.Cu") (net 12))
 (segment (start 149.102 47.4154) (end 121.3896 47.4154) (width 0.25) (layer "F.Cu") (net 12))
 (via (at 158.2148 47.4154) (size 0.6) (drill 0.4) (layers "F.Cu" "B.Cu") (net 12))
 (segment (start 157.2275 54.1708) (end 157.46 54.4033) (width 0.25) (layer "B.Cu") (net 12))
 (segment (start 157.46 54.4048) (end 157.5581 54.3067) (width 0.25) (layer "B.Cu") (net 12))
 (segment (start 157.2275 48.4027) (end 157.2275 54.1708) (width 0.25) (layer "B.Cu") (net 12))
 (segment (start 158.2148 47.4154) (end 157.9813 47.1819) (width 0.25) (layer "B.Cu") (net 12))
 (segment (start 157.5581 54.3067) (end 160.4736 54.3067) (width 0.25) (layer "B.Cu") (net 12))
 (segment (start 157.46 56) (end 157.46 54.5166) (width 0.25) (layer "B.Cu") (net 12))
 (segment (start 157.46 54.4048) (end 157.46 54.4033) (width 0.25) (layer "B.Cu") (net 12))
 (segment (start 157.9813 47.1819) (end 158.2148 47.4154) (width 0.25) (layer "B.Cu") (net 12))
 (segment (start 160.4736 54.3067) (end 163.5 57.3331) (width 0.25) (layer "B.Cu") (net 12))
 (segment (start 157.46 54.5166) (end 157.46 54.4048) (width 0.25) (layer "B.Cu") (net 12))
 (segment (start 163.5 57.3331) (end 163.5 97.46) (width 0.25) (layer "B.Cu") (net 12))
 (segment (start 158.2148 47.4154) (end 157.2275 48.4027) (width 0.25) (layer "B.Cu") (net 12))
 (segment (start 115.4162 52.4612) (end 114.0133 53.8641) (width 0.25) (layer "F.Cu") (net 11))
 (segment (start 157.9179 58.0821) (end 160 56) (width 0.25) (layer "F.Cu") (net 11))
 (segment (start 121.336 49.2) (end 118.0748 52.4612) (width 0.25) (layer "F.Cu") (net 11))
 (segment (start 114.0133 53.8641) (end 114.0133 56.1653) (width 0.25) (layer "F.Cu") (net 11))
 (segment (start 115.9301 58.0821) (end 157.9179 58.0821) (width 0.25) (layer "F.Cu") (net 11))
 (segment (start 118.0748 52.4612) (end 115.4162 52.4612) (width 0.25) (layer "F.Cu") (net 11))
 (segment (start 114.0133 56.1653) (end 115.9301 58.0821) (width 0.25) (layer "F.Cu") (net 11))
 (segment (start 160.96 97.46) (end 160.96 58.5567) (width 0.25) (layer "B.Cu") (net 11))
 (segment (start 160.96 58.5567) (end 160 57.5967) (width 0.25) (layer "B.Cu") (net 11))
 (segment (start 160 56) (end 160 57.5967) (width 0.25) (layer "B.Cu") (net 11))
 (segment (start 121.6685 50.447) (end 118.9062 53.2093) (width 0.25) (layer "F.Cu") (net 25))
 (segment (start 156.7135 47.4935) (end 149.6627 47.4935) (width 0.25) (layer "F.Cu") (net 25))
 (segment (start 149.3981 47.7581) (end 149.211 47.9452) (width 0.25) (layer "F.Cu") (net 25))
 (segment (start 158.42 49.2) (end 156.7135 47.4935) (width 0.25) (layer "F.Cu") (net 25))
 (segment (start 149.211 47.9452) (end 144.6047 47.9452) (width 0.25) (layer "F.Cu") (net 25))
 (segment (start 117.1307 53.2093) (end 115.34 55) (width 0.25) (layer "F.Cu") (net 25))
 (segment (start 149.3981 47.7581) (end 149.211 47.9452) (width 0.25) (layer "F.Cu") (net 25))
 (segment (start 149.6627 47.4935) (end 149.3981 47.7581) (width 0.25) (layer "F.Cu") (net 25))
 (segment (start 144.6047 47.9452) (end 142.1029 50.447) (width 0.25) (layer "F.Cu") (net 25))
 (segment (start 142.1029 50.447) (end 121.6685 50.447) (width 0.25) (layer "F.Cu") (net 25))
 (segment (start 118.9062 53.2093) (end 117.1307 53.2093) (width 0.25) (layer "F.Cu") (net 25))
 (segment (start 148.2307 51.7693) (end 150.8 49.2) (width 0.25) (layer "F.Cu") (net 22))
 (segment (start 123.6507 51.7693) (end 148.2307 51.7693) (width 0.25) (layer "F.Cu") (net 22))
 (segment (start 120.42 55) (end 123.6507 51.7693) (width 0.25) (layer "F.Cu") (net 22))
 (segment (start 149.4367 48.8393) (end 149.4367 49.806) (width 0.25) (layer "F.Cu") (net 23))
 (segment (start 121.9813 50.8987) (end 117.88 55) (width 0.25) (layer "F.Cu") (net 23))
 (segment (start 149.4367 49.806) (end 148.344 50.8987) (width 0.25) (layer "F.Cu") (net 23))
 (segment (start 148.344 50.8987) (end 121.9813 50.8987) (width 0.25) (layer "F.Cu") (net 23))
 (segment (start 152.1415 48.0015) (end 150.2745 48.0015) (width 0.25) (layer "F.Cu") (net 23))
 (segment (start 150.2745 48.0015) (end 149.4367 48.8393) (width 0.25) (layer "F.Cu") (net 23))
 (segment (start 153.34 49.2) (end 152.1415 48.0015) (width 0.25) (layer "F.Cu") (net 23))
 (segment (start 148.818 75.6574) (end 135.9226 75.6574) (width 0.25) (layer "F.Cu") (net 28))
 (segment (start 149.0036 75.4718) (end 148.818 75.6574) (width 0.25) (layer "F.Cu") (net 28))
 (segment (start 149.2682 75.2072) (end 149.0036 75.4718) (width 0.25) (layer "F.Cu") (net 28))
 (segment (start 152.6403 75.2072) (end 149.2682 75.2072) (width 0.25) (layer "F.Cu") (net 28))
 (segment (start 155.2243 77.7912) (end 152.6403 75.2072) (width 0.25) (layer "F.Cu") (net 28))
 (segment (start 149.0036 75.4718) (end 148.818 75.6574) (width 0.25) (layer "F.Cu") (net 28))
 (segment (start 135.9226 75.6574) (end 134.5 77.08) (width 0.25) (layer "F.Cu") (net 28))
 (via (at 155.2243 77.7912) (size 0.6) (drill 0.4) (layers "F.Cu" "B.Cu") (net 28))
 (segment (start 134.5 77.08) (end 133.08 77.08) (width 0.25) (layer "B.Cu") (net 28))
 (segment (start 133.08 77.08) (end 128 72) (width 0.25) (layer "B.Cu") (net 28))
 (segment (start 153.092 75.6589) (end 155.2243 77.7912) (width 0.25) (layer "B.Cu") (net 28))
 (segment (start 155.2243 87.8043) (end 158 90.58) (width 0.25) (layer "B.Cu") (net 28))
 (segment (start 155.2243 77.7912) (end 155.2243 87.8043) (width 0.25) (layer "B.Cu") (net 28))
 (segment (start 155.2243 77.7912) (end 153.092 75.6589) (width 0.25) (layer "B.Cu") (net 28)))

